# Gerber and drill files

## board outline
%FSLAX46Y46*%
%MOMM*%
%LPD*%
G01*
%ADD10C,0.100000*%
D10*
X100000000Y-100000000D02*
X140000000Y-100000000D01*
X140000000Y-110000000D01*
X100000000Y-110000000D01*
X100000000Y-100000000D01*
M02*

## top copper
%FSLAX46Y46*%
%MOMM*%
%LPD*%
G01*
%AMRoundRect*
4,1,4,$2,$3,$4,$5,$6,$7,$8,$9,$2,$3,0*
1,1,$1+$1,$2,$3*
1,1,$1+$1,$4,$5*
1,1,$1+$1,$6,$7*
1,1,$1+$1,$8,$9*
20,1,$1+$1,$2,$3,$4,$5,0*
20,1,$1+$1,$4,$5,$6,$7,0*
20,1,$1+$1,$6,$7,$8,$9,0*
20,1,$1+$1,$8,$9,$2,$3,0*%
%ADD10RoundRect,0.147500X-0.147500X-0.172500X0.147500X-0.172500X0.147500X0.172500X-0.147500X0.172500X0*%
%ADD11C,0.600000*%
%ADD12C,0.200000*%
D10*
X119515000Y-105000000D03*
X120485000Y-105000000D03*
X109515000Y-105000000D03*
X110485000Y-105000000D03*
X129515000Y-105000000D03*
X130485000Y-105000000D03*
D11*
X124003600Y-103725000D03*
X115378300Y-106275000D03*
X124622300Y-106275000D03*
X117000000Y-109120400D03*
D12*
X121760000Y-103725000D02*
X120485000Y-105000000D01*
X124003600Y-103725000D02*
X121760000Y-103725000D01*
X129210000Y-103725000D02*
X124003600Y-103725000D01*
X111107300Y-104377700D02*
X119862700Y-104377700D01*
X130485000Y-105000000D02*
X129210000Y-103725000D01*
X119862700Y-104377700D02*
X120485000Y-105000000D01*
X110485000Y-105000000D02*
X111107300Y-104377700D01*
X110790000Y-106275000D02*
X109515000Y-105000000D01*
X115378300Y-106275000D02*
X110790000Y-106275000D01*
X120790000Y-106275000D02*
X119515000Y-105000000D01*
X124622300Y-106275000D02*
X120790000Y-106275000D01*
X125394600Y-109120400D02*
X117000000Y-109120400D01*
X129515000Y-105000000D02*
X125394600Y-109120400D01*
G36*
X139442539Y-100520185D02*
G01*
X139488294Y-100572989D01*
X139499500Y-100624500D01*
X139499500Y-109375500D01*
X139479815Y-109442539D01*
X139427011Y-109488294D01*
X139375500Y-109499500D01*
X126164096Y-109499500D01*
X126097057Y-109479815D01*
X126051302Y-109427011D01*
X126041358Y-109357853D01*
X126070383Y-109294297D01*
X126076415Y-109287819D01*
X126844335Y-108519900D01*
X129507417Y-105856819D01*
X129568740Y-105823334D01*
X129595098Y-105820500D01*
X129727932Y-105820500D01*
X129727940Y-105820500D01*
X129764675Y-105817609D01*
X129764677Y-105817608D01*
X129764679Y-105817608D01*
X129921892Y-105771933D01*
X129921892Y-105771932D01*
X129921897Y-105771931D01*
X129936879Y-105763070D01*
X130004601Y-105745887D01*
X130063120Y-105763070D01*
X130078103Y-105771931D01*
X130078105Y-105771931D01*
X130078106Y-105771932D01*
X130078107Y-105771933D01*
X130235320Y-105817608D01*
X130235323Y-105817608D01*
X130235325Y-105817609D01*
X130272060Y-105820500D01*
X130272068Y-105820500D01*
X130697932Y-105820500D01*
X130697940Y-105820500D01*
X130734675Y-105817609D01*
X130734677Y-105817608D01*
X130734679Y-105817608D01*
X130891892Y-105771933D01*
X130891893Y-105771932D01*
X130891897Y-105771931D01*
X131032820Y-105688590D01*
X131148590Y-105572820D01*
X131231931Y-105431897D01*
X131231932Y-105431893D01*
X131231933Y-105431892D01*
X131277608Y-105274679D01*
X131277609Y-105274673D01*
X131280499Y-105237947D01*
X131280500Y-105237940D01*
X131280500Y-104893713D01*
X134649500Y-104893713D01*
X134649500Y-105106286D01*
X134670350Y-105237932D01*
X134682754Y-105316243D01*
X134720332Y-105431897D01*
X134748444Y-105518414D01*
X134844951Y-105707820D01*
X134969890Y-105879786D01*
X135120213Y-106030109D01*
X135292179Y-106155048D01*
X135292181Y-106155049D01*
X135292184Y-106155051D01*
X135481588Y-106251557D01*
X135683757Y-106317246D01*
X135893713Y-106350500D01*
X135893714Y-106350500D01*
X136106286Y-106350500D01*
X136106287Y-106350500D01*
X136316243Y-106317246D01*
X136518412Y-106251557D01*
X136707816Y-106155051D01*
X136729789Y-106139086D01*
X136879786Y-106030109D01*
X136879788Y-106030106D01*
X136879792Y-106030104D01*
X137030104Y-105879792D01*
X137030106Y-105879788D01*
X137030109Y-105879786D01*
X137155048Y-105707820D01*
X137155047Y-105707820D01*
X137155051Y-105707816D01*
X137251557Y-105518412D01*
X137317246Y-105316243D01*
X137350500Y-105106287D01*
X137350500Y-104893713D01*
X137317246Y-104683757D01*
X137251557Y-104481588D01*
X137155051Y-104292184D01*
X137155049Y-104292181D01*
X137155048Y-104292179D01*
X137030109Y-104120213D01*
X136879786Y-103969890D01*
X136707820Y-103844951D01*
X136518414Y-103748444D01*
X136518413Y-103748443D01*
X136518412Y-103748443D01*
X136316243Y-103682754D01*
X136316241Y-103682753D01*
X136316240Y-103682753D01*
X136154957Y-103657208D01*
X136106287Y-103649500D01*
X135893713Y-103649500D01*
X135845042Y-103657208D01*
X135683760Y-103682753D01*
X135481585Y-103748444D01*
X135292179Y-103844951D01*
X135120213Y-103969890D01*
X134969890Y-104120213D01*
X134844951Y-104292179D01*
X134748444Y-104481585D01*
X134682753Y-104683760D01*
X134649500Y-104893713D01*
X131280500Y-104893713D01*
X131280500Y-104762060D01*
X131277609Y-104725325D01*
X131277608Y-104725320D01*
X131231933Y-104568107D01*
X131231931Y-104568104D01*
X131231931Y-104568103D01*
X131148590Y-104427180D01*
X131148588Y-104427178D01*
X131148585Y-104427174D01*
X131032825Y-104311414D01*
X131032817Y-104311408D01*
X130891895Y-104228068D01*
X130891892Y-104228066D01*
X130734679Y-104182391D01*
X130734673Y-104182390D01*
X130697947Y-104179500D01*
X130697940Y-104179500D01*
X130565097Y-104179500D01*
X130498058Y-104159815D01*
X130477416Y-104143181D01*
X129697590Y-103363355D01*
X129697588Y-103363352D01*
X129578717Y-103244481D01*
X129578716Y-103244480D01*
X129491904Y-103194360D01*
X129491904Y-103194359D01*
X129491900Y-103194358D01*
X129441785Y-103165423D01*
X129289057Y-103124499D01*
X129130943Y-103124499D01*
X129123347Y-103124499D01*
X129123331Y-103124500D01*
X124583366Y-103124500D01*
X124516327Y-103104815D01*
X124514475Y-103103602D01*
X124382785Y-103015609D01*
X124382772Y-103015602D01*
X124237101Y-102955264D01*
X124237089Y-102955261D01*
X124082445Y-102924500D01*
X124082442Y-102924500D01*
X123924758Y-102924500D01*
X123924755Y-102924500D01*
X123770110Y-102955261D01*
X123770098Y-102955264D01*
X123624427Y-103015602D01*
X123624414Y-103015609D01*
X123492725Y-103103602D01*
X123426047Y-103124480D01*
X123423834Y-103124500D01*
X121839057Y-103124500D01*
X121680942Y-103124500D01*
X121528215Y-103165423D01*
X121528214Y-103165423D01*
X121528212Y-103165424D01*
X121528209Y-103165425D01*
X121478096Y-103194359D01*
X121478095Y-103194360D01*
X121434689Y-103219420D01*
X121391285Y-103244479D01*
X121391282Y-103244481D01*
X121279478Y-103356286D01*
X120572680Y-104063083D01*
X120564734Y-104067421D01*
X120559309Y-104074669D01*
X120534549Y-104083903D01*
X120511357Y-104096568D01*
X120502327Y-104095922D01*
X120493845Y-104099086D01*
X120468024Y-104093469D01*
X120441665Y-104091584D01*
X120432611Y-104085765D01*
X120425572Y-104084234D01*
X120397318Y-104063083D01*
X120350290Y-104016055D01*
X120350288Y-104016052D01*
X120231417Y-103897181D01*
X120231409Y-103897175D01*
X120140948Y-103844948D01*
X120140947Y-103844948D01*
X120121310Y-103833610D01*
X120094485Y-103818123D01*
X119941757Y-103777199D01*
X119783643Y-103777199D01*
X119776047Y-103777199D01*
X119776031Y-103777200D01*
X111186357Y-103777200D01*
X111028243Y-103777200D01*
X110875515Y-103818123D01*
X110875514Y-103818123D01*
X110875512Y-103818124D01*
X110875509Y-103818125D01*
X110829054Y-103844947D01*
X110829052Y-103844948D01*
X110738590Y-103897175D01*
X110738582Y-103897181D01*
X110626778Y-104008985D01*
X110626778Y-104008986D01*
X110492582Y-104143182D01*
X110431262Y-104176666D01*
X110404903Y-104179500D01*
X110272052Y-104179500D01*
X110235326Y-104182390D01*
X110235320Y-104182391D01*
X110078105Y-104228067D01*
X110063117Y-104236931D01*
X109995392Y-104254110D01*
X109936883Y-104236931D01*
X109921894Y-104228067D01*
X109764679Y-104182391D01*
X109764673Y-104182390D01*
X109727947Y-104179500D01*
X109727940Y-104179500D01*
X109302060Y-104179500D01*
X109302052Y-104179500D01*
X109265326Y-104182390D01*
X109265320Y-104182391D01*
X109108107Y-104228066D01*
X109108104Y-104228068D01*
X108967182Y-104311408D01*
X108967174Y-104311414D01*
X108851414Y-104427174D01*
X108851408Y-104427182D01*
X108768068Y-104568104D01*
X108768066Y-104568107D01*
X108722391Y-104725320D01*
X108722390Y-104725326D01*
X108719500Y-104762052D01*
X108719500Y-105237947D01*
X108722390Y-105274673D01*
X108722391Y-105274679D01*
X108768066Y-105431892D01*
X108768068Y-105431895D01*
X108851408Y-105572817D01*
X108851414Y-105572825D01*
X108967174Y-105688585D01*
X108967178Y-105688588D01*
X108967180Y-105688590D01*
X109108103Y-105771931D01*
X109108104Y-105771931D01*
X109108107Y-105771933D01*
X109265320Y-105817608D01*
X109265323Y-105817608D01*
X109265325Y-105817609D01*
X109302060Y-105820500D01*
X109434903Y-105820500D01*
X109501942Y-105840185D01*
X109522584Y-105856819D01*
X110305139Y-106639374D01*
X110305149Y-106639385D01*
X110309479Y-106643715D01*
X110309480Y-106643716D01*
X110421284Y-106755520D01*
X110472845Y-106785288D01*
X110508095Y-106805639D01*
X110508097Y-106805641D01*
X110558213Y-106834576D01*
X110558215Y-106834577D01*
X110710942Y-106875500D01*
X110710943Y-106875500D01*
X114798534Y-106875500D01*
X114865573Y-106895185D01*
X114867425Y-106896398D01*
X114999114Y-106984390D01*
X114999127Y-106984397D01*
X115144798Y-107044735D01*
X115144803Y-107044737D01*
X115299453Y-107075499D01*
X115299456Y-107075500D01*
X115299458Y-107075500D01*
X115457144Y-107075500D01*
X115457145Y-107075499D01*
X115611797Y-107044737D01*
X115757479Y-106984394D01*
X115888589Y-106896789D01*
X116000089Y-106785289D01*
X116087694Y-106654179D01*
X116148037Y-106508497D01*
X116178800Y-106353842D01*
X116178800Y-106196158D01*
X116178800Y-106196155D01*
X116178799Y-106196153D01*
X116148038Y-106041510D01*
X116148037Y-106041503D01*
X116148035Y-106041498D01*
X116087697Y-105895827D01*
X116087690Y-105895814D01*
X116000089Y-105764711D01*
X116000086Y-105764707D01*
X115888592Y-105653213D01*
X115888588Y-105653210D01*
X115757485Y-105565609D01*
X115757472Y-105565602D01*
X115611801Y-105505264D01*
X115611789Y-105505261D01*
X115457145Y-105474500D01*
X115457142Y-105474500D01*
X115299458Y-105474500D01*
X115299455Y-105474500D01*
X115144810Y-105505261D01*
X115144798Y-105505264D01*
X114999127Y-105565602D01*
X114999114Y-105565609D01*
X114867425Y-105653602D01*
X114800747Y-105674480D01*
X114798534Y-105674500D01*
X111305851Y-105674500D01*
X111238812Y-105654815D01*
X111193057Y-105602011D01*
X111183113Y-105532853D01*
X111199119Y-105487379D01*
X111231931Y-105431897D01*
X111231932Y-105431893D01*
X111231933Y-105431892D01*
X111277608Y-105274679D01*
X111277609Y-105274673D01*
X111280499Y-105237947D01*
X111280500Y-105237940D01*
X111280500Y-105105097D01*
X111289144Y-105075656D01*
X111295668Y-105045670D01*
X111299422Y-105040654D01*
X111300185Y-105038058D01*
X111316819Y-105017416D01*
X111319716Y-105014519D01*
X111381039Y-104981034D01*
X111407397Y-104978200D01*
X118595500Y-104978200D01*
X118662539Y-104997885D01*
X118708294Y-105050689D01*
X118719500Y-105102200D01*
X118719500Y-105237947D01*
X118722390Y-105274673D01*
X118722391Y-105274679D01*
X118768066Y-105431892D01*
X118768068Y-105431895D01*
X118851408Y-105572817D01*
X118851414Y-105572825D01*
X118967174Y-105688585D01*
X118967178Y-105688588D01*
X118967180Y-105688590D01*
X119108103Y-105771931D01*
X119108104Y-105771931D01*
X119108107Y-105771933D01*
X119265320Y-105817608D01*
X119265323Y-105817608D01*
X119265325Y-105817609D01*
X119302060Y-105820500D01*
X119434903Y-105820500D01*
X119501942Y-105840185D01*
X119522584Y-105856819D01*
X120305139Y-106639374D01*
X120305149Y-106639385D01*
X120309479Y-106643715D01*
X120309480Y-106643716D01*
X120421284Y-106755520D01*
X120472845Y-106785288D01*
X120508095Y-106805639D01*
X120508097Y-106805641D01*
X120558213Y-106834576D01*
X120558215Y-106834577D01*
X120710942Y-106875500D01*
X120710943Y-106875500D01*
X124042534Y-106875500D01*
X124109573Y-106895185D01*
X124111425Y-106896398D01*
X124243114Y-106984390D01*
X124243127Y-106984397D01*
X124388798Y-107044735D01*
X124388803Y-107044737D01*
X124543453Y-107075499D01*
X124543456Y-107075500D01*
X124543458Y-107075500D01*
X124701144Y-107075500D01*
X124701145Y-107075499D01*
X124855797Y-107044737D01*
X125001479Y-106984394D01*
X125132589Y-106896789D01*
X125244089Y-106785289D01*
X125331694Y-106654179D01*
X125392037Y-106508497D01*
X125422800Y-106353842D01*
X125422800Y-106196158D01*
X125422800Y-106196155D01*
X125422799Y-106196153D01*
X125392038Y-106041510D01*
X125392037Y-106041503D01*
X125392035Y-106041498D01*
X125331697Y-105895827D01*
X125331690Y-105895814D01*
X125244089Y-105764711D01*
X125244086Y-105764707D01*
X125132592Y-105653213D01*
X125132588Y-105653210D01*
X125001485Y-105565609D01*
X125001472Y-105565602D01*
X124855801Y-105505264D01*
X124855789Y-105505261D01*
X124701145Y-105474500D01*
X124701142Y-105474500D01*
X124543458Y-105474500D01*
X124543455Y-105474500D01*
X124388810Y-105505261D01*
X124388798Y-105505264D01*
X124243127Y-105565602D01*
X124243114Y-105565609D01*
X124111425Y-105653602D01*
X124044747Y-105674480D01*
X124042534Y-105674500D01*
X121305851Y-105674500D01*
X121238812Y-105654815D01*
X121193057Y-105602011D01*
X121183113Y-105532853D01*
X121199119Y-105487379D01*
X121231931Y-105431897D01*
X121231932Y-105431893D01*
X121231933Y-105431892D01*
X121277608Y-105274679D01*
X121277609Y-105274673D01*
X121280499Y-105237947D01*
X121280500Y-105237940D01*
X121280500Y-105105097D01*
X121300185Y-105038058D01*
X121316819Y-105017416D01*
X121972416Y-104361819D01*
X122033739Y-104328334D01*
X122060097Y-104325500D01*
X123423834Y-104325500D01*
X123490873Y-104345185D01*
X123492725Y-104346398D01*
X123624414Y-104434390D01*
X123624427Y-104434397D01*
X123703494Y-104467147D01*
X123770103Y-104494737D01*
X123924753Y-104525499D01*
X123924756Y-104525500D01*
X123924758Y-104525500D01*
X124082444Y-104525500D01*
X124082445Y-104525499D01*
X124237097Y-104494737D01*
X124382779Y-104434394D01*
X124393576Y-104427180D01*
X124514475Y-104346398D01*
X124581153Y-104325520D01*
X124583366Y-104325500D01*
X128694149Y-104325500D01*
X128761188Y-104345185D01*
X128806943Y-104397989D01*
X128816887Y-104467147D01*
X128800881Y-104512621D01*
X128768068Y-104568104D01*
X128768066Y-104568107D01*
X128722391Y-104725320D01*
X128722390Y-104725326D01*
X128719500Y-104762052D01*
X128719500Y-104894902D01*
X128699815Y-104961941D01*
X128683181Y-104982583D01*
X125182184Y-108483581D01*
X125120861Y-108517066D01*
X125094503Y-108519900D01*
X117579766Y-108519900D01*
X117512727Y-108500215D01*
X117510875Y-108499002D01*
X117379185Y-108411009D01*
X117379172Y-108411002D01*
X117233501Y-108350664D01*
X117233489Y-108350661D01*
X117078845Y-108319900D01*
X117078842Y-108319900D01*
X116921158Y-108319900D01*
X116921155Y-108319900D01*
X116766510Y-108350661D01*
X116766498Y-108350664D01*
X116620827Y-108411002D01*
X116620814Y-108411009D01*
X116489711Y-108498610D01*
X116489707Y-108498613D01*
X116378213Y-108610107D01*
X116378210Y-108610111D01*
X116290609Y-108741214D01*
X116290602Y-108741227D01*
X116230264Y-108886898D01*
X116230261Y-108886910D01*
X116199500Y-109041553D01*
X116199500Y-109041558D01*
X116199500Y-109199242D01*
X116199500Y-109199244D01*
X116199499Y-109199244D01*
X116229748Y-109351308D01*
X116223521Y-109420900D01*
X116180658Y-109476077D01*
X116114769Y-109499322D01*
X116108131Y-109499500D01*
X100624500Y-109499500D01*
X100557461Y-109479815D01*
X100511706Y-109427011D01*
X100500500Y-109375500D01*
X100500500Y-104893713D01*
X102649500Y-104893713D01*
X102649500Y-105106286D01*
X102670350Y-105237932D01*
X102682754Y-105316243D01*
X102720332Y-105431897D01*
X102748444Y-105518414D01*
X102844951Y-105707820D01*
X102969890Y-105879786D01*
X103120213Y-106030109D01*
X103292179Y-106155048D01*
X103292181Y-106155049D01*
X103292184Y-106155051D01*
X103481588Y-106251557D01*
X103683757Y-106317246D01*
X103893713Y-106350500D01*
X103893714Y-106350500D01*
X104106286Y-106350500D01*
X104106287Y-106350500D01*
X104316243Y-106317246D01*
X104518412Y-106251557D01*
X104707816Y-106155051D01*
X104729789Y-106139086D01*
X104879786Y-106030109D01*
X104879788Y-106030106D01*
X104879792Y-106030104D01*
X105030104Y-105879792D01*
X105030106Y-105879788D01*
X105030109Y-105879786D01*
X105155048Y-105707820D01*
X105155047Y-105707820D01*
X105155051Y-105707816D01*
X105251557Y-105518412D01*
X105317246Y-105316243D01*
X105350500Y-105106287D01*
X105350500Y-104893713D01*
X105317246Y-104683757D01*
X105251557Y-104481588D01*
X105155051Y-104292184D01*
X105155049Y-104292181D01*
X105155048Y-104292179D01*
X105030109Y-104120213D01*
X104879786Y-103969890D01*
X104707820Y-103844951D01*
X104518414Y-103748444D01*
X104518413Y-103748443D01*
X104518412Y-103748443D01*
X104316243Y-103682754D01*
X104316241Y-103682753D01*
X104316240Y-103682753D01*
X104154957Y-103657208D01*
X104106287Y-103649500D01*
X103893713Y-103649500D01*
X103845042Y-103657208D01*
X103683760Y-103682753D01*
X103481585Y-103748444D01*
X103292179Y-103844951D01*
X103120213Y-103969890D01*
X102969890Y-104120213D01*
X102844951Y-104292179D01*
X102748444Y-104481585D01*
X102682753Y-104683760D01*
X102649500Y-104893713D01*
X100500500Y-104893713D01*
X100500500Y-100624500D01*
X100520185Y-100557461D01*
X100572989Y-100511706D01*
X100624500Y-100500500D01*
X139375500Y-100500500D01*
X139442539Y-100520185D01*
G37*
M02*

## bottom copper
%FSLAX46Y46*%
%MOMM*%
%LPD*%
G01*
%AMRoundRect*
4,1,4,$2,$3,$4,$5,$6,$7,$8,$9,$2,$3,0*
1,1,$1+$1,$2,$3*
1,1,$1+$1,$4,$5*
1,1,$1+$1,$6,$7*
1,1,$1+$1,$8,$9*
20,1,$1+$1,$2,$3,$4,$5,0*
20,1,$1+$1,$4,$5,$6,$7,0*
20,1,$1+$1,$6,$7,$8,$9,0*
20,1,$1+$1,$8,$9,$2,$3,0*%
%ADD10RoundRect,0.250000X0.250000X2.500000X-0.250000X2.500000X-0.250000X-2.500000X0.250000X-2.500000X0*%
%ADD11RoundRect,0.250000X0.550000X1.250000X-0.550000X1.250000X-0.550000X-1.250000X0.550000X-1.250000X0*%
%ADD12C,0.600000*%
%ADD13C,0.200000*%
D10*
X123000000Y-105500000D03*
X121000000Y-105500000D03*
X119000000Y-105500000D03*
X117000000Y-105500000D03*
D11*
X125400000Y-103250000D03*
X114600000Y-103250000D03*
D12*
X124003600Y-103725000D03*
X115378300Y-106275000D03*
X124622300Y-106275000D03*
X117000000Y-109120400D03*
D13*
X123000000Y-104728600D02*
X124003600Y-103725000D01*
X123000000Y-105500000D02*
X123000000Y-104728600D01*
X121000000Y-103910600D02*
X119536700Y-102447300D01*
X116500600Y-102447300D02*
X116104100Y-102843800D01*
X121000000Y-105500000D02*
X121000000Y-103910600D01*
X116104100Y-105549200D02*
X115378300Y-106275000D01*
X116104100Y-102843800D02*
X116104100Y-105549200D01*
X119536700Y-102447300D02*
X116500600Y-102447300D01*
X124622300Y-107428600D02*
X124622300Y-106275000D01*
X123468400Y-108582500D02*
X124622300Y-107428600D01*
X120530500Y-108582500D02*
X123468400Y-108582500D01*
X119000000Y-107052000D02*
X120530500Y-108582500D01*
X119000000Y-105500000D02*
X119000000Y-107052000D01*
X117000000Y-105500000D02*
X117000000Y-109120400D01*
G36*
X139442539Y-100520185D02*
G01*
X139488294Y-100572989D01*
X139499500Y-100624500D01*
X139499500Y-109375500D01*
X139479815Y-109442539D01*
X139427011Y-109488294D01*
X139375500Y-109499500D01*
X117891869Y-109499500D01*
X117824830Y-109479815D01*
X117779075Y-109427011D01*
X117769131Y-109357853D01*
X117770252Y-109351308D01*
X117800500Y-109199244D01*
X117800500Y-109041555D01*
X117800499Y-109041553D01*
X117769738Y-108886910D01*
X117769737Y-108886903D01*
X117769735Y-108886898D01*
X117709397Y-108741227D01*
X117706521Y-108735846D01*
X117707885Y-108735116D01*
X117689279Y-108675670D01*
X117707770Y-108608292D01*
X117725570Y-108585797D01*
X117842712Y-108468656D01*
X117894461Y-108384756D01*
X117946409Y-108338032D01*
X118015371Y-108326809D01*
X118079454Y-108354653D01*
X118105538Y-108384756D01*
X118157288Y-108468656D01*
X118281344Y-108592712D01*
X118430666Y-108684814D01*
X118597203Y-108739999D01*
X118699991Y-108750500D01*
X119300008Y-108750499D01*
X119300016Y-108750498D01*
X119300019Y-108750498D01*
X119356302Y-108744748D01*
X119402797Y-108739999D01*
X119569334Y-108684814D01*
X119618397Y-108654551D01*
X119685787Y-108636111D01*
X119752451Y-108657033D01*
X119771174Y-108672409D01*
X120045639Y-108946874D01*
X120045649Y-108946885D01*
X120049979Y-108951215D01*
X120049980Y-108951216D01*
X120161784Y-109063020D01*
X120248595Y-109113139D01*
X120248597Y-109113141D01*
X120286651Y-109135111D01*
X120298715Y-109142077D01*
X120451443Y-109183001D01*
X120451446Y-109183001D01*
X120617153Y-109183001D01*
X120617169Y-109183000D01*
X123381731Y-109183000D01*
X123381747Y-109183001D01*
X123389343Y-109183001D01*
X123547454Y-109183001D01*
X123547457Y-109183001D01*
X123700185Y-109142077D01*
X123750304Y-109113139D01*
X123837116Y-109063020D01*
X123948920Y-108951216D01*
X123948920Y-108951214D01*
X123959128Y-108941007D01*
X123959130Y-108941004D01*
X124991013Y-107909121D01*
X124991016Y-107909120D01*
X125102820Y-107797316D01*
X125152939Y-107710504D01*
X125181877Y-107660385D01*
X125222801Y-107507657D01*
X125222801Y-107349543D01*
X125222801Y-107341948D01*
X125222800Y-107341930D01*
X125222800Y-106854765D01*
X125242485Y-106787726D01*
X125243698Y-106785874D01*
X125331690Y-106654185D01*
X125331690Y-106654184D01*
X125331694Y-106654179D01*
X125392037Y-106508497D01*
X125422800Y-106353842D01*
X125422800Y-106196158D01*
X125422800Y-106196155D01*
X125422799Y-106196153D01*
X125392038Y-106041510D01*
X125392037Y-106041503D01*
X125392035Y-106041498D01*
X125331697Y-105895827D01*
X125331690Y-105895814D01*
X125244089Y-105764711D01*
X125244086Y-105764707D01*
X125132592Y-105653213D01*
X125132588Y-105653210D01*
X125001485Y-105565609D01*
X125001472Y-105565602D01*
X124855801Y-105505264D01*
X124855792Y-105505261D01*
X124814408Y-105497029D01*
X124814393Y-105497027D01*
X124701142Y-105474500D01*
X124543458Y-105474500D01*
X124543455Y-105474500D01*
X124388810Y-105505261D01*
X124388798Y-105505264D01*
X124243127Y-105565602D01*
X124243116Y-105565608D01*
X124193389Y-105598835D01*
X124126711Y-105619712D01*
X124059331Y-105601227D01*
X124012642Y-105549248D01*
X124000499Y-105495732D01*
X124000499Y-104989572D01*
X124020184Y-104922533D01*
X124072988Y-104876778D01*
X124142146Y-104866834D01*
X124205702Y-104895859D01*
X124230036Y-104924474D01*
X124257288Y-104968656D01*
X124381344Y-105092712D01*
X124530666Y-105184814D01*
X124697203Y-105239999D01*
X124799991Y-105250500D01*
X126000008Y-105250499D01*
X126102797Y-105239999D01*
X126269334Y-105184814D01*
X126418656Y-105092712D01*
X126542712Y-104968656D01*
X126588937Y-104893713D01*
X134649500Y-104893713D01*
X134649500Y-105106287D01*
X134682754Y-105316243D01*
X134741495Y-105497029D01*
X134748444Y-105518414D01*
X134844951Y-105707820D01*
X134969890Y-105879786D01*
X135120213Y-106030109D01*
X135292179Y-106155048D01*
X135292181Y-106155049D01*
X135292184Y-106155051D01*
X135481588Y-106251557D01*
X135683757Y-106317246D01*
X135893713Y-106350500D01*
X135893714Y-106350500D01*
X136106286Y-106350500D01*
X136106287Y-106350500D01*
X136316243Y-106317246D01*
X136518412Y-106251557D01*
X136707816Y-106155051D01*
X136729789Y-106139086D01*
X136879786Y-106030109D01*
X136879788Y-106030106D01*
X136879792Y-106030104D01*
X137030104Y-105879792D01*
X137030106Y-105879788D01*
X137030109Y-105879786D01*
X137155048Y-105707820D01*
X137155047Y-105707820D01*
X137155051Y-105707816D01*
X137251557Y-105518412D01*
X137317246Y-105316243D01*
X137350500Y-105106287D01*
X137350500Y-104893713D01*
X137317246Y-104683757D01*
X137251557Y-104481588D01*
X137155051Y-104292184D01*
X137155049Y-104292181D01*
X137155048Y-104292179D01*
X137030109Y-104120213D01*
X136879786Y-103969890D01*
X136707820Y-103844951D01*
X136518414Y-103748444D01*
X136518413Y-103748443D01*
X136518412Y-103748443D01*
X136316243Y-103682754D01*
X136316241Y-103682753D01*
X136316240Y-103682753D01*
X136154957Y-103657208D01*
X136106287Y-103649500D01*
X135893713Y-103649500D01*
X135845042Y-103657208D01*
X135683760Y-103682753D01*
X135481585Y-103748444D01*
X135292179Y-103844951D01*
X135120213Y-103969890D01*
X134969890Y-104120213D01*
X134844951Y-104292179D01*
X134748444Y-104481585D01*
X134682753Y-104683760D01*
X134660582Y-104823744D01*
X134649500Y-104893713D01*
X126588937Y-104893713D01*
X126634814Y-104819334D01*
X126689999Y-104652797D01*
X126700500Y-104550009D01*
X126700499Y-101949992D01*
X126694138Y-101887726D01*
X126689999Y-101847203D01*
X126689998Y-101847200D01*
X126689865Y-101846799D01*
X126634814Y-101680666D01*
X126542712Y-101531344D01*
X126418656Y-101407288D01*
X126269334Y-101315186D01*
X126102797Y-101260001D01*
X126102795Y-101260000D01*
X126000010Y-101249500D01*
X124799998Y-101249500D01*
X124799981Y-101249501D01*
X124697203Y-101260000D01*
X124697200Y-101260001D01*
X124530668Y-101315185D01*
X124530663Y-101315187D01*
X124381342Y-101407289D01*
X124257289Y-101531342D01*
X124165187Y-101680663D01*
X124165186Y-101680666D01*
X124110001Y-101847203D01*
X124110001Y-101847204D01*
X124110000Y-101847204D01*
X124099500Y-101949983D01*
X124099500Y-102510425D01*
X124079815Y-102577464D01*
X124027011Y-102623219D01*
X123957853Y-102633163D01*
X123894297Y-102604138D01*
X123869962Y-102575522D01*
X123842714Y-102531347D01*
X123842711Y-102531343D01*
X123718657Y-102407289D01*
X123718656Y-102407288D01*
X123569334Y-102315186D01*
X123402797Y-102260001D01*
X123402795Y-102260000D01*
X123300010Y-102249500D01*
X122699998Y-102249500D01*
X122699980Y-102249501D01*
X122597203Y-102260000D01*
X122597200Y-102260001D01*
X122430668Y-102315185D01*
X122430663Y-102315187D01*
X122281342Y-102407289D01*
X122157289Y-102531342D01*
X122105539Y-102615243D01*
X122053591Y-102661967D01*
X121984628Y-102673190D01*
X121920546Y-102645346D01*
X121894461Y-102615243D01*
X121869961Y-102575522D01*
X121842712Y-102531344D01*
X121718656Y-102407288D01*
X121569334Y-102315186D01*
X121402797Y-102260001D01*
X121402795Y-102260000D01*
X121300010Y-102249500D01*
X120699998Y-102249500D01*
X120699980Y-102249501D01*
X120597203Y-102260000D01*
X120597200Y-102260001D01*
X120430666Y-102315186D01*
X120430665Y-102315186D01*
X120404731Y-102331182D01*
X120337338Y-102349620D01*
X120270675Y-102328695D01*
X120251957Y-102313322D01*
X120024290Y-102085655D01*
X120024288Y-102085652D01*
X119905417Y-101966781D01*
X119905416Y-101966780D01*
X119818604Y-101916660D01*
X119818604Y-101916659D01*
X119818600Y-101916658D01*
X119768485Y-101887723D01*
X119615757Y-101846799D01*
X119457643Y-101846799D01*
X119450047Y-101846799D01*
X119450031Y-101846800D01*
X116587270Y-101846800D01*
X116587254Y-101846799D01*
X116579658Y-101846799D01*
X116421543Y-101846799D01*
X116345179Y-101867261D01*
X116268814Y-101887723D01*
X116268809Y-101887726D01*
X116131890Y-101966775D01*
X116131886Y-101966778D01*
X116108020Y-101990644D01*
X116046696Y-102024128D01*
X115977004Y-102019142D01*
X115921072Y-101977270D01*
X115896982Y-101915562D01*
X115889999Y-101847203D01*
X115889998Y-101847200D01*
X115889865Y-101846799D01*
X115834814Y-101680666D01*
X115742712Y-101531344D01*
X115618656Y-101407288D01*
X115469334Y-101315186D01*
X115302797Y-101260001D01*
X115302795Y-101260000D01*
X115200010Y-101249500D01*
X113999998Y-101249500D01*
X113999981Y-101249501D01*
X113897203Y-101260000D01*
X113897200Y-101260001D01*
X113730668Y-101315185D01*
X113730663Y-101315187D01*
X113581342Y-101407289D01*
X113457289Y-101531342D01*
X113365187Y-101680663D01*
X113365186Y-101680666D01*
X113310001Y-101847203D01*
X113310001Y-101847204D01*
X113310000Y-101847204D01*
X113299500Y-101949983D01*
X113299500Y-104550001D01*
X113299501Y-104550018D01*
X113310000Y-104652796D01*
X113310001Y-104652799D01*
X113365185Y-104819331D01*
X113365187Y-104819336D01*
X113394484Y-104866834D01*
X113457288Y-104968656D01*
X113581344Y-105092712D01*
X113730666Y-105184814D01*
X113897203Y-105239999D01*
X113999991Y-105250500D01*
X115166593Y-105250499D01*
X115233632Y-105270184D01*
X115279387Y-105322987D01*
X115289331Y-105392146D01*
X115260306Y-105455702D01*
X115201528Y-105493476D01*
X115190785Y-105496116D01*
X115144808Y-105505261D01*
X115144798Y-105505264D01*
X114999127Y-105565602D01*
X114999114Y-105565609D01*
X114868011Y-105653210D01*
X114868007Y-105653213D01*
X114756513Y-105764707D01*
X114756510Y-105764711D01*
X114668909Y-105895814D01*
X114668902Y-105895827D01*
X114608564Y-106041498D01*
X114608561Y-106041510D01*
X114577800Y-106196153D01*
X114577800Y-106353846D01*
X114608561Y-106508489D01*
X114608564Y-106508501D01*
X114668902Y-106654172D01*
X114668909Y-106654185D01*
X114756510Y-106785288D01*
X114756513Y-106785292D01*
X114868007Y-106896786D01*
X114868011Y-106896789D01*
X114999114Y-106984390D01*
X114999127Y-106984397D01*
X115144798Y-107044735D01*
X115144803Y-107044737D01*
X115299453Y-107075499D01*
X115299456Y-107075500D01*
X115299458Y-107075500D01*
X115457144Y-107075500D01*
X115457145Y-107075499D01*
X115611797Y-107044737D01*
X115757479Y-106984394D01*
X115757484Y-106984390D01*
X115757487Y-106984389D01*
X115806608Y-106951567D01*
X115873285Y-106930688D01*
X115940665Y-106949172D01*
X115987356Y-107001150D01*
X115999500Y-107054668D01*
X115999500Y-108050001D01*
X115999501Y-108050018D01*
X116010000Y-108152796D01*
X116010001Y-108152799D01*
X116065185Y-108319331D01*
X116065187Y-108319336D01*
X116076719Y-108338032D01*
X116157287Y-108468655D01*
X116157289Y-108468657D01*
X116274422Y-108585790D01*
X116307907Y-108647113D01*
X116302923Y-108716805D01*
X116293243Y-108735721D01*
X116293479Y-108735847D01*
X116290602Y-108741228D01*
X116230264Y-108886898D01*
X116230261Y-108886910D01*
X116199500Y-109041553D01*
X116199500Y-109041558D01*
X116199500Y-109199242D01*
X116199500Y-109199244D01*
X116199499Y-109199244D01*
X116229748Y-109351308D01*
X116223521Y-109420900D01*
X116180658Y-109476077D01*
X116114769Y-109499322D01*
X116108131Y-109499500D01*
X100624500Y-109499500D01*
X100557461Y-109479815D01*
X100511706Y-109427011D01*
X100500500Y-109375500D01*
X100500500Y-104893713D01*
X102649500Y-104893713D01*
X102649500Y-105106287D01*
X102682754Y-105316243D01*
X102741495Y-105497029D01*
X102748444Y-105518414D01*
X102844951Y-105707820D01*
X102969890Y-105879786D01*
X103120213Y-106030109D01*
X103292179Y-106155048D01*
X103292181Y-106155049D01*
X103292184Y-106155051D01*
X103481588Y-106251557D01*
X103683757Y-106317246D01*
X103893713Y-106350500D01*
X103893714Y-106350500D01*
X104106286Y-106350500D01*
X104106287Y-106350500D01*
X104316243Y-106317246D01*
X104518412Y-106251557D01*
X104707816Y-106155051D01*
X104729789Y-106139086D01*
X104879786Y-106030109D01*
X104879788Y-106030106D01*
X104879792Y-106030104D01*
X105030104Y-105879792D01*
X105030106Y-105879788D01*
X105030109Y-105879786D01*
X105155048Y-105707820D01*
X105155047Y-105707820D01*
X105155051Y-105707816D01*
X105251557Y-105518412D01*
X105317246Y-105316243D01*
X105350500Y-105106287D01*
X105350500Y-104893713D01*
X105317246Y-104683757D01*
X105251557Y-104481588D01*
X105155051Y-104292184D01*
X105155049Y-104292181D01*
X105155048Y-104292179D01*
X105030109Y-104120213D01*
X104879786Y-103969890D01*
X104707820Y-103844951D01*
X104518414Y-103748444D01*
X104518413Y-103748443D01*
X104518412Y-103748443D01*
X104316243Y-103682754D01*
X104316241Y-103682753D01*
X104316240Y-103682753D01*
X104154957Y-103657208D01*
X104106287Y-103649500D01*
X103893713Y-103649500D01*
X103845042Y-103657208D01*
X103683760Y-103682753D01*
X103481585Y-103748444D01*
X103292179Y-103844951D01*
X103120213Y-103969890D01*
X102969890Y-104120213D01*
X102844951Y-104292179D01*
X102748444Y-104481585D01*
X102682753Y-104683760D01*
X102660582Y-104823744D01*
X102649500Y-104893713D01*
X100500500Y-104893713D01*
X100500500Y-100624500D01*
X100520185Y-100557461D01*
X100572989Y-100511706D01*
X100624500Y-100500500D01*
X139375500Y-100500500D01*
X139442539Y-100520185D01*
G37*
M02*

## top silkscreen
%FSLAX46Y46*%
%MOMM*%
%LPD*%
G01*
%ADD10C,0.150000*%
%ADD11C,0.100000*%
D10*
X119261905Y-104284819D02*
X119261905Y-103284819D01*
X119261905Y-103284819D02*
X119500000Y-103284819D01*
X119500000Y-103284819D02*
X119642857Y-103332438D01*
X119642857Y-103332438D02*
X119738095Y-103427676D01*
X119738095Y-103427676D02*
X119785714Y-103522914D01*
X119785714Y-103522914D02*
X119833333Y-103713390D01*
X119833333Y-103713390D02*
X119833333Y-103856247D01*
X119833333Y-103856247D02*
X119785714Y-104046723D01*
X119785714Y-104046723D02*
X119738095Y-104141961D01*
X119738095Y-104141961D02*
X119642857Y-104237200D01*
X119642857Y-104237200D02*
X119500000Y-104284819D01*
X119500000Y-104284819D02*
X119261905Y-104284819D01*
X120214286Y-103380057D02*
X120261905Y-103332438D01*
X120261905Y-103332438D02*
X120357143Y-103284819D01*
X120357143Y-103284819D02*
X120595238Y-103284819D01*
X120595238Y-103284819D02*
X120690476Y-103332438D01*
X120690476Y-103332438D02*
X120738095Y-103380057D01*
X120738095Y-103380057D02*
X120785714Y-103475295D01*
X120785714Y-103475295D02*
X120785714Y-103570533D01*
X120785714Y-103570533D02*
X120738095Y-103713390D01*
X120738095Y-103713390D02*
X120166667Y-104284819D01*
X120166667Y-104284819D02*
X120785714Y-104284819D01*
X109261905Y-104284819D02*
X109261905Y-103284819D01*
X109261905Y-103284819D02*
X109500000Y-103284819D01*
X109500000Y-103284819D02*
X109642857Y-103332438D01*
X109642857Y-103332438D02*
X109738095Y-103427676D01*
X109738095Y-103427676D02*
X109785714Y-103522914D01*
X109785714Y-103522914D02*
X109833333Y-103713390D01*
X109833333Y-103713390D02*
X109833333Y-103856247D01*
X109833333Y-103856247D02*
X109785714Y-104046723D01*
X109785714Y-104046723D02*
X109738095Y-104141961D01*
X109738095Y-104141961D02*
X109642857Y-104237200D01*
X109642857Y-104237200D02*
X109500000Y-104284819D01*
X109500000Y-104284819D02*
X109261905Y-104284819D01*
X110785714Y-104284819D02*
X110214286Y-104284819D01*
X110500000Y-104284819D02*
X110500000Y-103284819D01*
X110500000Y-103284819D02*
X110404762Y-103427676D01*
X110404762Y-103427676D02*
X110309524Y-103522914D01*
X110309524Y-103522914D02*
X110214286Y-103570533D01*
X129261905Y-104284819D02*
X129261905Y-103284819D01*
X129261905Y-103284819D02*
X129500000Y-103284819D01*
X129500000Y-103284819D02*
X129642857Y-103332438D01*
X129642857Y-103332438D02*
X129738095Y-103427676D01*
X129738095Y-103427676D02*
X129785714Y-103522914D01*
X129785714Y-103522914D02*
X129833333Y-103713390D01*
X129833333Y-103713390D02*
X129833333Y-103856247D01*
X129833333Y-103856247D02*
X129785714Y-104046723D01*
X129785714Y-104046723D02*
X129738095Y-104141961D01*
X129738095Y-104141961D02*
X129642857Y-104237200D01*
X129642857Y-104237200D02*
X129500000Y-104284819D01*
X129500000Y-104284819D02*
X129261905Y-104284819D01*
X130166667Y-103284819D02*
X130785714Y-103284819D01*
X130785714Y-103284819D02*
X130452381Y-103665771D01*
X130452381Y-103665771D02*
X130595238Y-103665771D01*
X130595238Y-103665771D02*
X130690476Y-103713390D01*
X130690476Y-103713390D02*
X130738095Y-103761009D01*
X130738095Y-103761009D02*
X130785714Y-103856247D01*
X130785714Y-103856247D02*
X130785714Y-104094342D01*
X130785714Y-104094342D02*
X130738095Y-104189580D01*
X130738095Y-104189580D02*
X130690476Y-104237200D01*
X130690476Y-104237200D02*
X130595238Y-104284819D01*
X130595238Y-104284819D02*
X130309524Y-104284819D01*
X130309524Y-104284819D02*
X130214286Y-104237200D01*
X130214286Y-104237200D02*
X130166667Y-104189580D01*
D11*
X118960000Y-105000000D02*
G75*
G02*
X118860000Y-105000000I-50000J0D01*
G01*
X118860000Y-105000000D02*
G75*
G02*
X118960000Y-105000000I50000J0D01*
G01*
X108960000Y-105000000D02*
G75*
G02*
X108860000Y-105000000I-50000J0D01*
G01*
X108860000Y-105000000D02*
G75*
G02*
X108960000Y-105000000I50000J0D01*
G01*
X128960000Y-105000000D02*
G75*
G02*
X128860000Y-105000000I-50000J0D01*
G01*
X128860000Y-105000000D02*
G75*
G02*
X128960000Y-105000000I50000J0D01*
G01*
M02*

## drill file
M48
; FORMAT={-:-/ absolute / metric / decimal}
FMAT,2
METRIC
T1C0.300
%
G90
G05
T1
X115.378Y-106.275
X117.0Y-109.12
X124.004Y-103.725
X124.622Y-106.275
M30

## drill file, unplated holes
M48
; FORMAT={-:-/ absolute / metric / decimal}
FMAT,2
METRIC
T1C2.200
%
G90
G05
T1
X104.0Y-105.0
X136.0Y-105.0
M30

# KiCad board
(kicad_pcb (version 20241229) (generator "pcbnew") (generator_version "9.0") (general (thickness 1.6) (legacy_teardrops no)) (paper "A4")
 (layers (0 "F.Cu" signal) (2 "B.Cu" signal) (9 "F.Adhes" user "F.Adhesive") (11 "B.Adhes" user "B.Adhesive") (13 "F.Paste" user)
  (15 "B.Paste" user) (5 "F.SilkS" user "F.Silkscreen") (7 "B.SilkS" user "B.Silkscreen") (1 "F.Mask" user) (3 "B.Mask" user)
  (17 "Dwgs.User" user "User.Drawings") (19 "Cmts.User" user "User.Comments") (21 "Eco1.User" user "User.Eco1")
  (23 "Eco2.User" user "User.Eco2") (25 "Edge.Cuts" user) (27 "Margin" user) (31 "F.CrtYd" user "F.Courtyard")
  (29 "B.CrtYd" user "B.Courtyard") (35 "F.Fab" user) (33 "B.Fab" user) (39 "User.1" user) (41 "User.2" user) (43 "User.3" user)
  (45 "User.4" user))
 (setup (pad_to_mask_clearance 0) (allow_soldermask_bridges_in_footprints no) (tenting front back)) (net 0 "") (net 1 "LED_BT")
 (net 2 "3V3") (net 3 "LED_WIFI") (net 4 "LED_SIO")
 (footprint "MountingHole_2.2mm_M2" (layer "F.Cu") (at 136 105)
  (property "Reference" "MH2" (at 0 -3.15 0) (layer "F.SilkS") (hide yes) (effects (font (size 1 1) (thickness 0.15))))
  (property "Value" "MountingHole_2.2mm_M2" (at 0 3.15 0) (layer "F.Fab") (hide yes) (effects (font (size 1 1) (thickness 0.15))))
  (pad "" np_thru_hole circle (at 0 0) (size 2.2 2.2) (drill 2.2) (layers "*.Cu" "*.Mask")))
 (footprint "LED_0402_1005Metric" (layer "F.Cu") (at 120 105)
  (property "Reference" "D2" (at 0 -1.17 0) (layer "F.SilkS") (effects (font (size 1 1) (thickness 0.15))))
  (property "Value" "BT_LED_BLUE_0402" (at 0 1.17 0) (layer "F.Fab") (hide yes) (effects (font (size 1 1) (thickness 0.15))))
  (fp_circle (center -1.09 0) (end -1.04 0) (stroke (width 0.1) (type solid)) (fill no) (layer "F.SilkS"))
  (pad "1" smd roundrect (at -0.485 0) (size 0.59 0.64) (layers "F.Cu" "F.Mask" "F.Paste") (roundrect_rratio 0.25) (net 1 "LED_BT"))
  (pad "2" smd roundrect (at 0.485 0) (size 0.59 0.64) (layers "F.Cu" "F.Mask" "F.Paste") (roundrect_rratio 0.25) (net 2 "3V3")))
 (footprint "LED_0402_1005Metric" (layer "F.Cu") (at 110 105)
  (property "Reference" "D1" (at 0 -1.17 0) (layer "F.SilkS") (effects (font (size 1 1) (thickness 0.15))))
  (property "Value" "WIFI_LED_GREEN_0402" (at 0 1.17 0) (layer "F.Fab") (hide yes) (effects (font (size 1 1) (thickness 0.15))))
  (fp_circle (center -1.09 0) (end -1.04 0) (stroke (width 0.1) (type solid)) (fill no) (layer "F.SilkS"))
  (pad "1" smd roundrect (at -0.485 0) (size 0.59 0.64) (layers "F.Cu" "F.Mask" "F.Paste") (roundrect_rratio 0.25) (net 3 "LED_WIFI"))
  (pad "2" smd roundrect (at 0.485 0) (size 0.59 0.64) (layers "F.Cu" "F.Mask" "F.Paste") (roundrect_rratio 0.25) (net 2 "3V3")))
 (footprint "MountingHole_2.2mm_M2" (layer "F.Cu") (at 104 105)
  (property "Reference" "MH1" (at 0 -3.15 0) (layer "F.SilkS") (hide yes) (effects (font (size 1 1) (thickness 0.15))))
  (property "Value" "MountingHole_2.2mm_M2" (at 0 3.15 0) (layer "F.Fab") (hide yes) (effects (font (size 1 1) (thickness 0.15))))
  (pad "" np_thru_hole circle (at 0 0) (size 2.2 2.2) (drill 2.2) (layers "*.Cu" "*.Mask")))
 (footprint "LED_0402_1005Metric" (layer "F.Cu") (at 130 105)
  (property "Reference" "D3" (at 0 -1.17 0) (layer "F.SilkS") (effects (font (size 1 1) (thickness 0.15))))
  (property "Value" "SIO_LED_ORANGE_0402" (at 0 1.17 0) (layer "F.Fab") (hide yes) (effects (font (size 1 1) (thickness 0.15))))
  (fp_circle (center -1.09 0) (end -1.04 0) (stroke (width 0.1) (type solid)) (fill no) (layer "F.SilkS"))
  (pad "1" smd roundrect (at -0.485 0) (size 0.59 0.64) (layers "F.Cu" "F.Mask" "F.Paste") (roundrect_rratio 0.25) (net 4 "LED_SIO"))
  (pad "2" smd roundrect (at 0.485 0) (size 0.59 0.64) (layers "F.Cu" "F.Mask" "F.Paste") (roundrect_rratio 0.25) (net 2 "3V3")))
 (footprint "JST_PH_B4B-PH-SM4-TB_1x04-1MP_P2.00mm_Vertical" (layer "B.Cu") (at 120 105 180)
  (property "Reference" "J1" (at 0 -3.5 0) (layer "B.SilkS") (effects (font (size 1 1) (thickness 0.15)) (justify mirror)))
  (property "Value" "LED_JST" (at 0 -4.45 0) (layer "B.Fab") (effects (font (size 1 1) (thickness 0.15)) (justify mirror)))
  (pad "1" smd roundrect (at -3 -0.5 180) (size 1 5.5) (layers "B.Cu" "B.Mask" "B.Paste") (roundrect_rratio 0.25) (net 2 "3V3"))
  (pad "2" smd roundrect (at -1 -0.5 180) (size 1 5.5) (layers "B.Cu" "B.Mask" "B.Paste") (roundrect_rratio 0.25) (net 3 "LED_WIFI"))
  (pad "3" smd roundrect (at 1 -0.5 180) (size 1 5.5) (layers "B.Cu" "B.Mask" "B.Paste") (roundrect_rratio 0.25) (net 1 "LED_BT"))
  (pad "4" smd roundrect (at 3 -0.5 180) (size 1 5.5) (layers "B.Cu" "B.Mask" "B.Paste") (roundrect_rratio 0.25) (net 4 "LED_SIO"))
  (pad "MP" smd roundrect (at -5.4 1.75 180) (size 1.6 3) (layers "B.Cu" "B.Mask" "B.Paste") (roundrect_rratio 0.15625))
  (pad "MP" smd roundrect (at 5.4 1.75 180) (size 1.6 3) (layers "B.Cu" "B.Mask" "B.Paste") (roundrect_rratio 0.15625)))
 (gr_rect (start 100 100) (end 140 110) (stroke (width 0.1) (type default)) (fill no) (layer "Edge.Cuts"))
 (segment (start 121.76 103.725) (end 120.485 105) (width 0.2) (layer "F.Cu") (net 2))
 (segment (start 124.0036 103.725) (end 121.76 103.725) (width 0.2) (layer "F.Cu") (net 2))
 (segment (start 129.21 103.725) (end 124.0036 103.725) (width 0.2) (layer "F.Cu") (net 2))
 (segment (start 111.1073 104.3777) (end 119.8627 104.3777) (width 0.2) (layer "F.Cu") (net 2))
 (segment (start 130.485 105) (end 129.21 103.725) (width 0.2) (layer "F.Cu") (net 2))
 (segment (start 119.8627 104.3777) (end 120.485 105) (width 0.2) (layer "F.Cu") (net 2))
 (segment (start 110.485 105) (end 111.1073 104.3777) (width 0.2) (layer "F.Cu") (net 2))
 (via (at 124.0036 103.725) (size 0.6) (drill 0.3) (layers "F.Cu" "B.Cu") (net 2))
 (segment (start 123 104.7286) (end 124.0036 103.725) (width 0.2) (layer "B.Cu") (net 2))
 (segment (start 123 105.5) (end 123 104.7286) (width 0.2) (layer "B.Cu") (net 2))
 (segment (start 110.79 106.275) (end 109.515 105) (width 0.2) (layer "F.Cu") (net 3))
 (segment (start 115.3783 106.275) (end 110.79 106.275) (width 0.2) (layer "F.Cu") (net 3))
 (via (at 115.3783 106.275) (size 0.6) (drill 0.3) (layers "F.Cu" "B.Cu") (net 3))
 (segment (start 121 103.9106) (end 119.5367 102.4473) (width 0.2) (layer "B.Cu") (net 3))
 (segment (start 116.5006 102.4473) (end 116.1041 102.8438) (width 0.2) (layer "B.Cu") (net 3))
 (segment (start 121 105.5) (end 121 103.9106) (width 0.2) (layer "B.Cu") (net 3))
 (segment (start 116.1041 105.5492) (end 115.3783 106.275) (width 0.2) (layer "B.Cu") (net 3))
 (segment (start 116.1041 102.8438) (end 116.1041 105.5492) (width 0.2) (layer "B.Cu") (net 3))
 (segment (start 119.5367 102.4473) (end 116.5006 102.4473) (width 0.2) (layer "B.Cu") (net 3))
 (segment (start 120.79 106.275) (end 119.515 105) (width 0.2) (layer "F.Cu") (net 1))
 (segment (start 124.6223 106.275) (end 120.79 106.275) (width 0.2) (layer "F.Cu") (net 1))
 (via (at 124.6223 106.275) (size 0.6) (drill 0.3) (layers "F.Cu" "B.Cu") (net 1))
 (segment (start 124.6223 107.4286) (end 124.6223 106.275) (width 0.2) (layer "B.Cu") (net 1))
 (segment (start 123.4684 108.5825) (end 124.6223 107.4286) (width 0.2) (layer "B.Cu") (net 1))
 (segment (start 120.5305 108.5825) (end 123.4684 108.5825) (width 0.2) (layer "B.Cu") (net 1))
 (segment (start 119 107.052) (end 120.5305 108.5825) (width 0.2) (layer "B.Cu") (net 1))
 (segment (start 119 105.5) (end 119 107.052) (width 0.2) (layer "B.Cu") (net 1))
 (segment (start 125.3946 109.1204) (end 117 109.1204) (width 0.2) (layer "F.Cu") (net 4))
 (segment (start 129.515 105) (end 125.3946 109.1204) (width 0.2) (layer "F.Cu") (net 4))
 (via (at 117 109.1204) (size 0.6) (drill 0.3) (layers "F.Cu" "B.Cu") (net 4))
 (segment (start 117 105.5) (end 117 109.1204) (width 0.2) (layer "B.Cu") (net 4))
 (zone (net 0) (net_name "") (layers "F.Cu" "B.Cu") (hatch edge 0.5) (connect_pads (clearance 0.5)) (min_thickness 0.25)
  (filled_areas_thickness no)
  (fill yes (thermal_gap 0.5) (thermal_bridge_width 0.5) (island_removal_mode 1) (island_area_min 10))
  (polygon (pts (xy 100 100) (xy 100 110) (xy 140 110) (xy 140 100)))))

